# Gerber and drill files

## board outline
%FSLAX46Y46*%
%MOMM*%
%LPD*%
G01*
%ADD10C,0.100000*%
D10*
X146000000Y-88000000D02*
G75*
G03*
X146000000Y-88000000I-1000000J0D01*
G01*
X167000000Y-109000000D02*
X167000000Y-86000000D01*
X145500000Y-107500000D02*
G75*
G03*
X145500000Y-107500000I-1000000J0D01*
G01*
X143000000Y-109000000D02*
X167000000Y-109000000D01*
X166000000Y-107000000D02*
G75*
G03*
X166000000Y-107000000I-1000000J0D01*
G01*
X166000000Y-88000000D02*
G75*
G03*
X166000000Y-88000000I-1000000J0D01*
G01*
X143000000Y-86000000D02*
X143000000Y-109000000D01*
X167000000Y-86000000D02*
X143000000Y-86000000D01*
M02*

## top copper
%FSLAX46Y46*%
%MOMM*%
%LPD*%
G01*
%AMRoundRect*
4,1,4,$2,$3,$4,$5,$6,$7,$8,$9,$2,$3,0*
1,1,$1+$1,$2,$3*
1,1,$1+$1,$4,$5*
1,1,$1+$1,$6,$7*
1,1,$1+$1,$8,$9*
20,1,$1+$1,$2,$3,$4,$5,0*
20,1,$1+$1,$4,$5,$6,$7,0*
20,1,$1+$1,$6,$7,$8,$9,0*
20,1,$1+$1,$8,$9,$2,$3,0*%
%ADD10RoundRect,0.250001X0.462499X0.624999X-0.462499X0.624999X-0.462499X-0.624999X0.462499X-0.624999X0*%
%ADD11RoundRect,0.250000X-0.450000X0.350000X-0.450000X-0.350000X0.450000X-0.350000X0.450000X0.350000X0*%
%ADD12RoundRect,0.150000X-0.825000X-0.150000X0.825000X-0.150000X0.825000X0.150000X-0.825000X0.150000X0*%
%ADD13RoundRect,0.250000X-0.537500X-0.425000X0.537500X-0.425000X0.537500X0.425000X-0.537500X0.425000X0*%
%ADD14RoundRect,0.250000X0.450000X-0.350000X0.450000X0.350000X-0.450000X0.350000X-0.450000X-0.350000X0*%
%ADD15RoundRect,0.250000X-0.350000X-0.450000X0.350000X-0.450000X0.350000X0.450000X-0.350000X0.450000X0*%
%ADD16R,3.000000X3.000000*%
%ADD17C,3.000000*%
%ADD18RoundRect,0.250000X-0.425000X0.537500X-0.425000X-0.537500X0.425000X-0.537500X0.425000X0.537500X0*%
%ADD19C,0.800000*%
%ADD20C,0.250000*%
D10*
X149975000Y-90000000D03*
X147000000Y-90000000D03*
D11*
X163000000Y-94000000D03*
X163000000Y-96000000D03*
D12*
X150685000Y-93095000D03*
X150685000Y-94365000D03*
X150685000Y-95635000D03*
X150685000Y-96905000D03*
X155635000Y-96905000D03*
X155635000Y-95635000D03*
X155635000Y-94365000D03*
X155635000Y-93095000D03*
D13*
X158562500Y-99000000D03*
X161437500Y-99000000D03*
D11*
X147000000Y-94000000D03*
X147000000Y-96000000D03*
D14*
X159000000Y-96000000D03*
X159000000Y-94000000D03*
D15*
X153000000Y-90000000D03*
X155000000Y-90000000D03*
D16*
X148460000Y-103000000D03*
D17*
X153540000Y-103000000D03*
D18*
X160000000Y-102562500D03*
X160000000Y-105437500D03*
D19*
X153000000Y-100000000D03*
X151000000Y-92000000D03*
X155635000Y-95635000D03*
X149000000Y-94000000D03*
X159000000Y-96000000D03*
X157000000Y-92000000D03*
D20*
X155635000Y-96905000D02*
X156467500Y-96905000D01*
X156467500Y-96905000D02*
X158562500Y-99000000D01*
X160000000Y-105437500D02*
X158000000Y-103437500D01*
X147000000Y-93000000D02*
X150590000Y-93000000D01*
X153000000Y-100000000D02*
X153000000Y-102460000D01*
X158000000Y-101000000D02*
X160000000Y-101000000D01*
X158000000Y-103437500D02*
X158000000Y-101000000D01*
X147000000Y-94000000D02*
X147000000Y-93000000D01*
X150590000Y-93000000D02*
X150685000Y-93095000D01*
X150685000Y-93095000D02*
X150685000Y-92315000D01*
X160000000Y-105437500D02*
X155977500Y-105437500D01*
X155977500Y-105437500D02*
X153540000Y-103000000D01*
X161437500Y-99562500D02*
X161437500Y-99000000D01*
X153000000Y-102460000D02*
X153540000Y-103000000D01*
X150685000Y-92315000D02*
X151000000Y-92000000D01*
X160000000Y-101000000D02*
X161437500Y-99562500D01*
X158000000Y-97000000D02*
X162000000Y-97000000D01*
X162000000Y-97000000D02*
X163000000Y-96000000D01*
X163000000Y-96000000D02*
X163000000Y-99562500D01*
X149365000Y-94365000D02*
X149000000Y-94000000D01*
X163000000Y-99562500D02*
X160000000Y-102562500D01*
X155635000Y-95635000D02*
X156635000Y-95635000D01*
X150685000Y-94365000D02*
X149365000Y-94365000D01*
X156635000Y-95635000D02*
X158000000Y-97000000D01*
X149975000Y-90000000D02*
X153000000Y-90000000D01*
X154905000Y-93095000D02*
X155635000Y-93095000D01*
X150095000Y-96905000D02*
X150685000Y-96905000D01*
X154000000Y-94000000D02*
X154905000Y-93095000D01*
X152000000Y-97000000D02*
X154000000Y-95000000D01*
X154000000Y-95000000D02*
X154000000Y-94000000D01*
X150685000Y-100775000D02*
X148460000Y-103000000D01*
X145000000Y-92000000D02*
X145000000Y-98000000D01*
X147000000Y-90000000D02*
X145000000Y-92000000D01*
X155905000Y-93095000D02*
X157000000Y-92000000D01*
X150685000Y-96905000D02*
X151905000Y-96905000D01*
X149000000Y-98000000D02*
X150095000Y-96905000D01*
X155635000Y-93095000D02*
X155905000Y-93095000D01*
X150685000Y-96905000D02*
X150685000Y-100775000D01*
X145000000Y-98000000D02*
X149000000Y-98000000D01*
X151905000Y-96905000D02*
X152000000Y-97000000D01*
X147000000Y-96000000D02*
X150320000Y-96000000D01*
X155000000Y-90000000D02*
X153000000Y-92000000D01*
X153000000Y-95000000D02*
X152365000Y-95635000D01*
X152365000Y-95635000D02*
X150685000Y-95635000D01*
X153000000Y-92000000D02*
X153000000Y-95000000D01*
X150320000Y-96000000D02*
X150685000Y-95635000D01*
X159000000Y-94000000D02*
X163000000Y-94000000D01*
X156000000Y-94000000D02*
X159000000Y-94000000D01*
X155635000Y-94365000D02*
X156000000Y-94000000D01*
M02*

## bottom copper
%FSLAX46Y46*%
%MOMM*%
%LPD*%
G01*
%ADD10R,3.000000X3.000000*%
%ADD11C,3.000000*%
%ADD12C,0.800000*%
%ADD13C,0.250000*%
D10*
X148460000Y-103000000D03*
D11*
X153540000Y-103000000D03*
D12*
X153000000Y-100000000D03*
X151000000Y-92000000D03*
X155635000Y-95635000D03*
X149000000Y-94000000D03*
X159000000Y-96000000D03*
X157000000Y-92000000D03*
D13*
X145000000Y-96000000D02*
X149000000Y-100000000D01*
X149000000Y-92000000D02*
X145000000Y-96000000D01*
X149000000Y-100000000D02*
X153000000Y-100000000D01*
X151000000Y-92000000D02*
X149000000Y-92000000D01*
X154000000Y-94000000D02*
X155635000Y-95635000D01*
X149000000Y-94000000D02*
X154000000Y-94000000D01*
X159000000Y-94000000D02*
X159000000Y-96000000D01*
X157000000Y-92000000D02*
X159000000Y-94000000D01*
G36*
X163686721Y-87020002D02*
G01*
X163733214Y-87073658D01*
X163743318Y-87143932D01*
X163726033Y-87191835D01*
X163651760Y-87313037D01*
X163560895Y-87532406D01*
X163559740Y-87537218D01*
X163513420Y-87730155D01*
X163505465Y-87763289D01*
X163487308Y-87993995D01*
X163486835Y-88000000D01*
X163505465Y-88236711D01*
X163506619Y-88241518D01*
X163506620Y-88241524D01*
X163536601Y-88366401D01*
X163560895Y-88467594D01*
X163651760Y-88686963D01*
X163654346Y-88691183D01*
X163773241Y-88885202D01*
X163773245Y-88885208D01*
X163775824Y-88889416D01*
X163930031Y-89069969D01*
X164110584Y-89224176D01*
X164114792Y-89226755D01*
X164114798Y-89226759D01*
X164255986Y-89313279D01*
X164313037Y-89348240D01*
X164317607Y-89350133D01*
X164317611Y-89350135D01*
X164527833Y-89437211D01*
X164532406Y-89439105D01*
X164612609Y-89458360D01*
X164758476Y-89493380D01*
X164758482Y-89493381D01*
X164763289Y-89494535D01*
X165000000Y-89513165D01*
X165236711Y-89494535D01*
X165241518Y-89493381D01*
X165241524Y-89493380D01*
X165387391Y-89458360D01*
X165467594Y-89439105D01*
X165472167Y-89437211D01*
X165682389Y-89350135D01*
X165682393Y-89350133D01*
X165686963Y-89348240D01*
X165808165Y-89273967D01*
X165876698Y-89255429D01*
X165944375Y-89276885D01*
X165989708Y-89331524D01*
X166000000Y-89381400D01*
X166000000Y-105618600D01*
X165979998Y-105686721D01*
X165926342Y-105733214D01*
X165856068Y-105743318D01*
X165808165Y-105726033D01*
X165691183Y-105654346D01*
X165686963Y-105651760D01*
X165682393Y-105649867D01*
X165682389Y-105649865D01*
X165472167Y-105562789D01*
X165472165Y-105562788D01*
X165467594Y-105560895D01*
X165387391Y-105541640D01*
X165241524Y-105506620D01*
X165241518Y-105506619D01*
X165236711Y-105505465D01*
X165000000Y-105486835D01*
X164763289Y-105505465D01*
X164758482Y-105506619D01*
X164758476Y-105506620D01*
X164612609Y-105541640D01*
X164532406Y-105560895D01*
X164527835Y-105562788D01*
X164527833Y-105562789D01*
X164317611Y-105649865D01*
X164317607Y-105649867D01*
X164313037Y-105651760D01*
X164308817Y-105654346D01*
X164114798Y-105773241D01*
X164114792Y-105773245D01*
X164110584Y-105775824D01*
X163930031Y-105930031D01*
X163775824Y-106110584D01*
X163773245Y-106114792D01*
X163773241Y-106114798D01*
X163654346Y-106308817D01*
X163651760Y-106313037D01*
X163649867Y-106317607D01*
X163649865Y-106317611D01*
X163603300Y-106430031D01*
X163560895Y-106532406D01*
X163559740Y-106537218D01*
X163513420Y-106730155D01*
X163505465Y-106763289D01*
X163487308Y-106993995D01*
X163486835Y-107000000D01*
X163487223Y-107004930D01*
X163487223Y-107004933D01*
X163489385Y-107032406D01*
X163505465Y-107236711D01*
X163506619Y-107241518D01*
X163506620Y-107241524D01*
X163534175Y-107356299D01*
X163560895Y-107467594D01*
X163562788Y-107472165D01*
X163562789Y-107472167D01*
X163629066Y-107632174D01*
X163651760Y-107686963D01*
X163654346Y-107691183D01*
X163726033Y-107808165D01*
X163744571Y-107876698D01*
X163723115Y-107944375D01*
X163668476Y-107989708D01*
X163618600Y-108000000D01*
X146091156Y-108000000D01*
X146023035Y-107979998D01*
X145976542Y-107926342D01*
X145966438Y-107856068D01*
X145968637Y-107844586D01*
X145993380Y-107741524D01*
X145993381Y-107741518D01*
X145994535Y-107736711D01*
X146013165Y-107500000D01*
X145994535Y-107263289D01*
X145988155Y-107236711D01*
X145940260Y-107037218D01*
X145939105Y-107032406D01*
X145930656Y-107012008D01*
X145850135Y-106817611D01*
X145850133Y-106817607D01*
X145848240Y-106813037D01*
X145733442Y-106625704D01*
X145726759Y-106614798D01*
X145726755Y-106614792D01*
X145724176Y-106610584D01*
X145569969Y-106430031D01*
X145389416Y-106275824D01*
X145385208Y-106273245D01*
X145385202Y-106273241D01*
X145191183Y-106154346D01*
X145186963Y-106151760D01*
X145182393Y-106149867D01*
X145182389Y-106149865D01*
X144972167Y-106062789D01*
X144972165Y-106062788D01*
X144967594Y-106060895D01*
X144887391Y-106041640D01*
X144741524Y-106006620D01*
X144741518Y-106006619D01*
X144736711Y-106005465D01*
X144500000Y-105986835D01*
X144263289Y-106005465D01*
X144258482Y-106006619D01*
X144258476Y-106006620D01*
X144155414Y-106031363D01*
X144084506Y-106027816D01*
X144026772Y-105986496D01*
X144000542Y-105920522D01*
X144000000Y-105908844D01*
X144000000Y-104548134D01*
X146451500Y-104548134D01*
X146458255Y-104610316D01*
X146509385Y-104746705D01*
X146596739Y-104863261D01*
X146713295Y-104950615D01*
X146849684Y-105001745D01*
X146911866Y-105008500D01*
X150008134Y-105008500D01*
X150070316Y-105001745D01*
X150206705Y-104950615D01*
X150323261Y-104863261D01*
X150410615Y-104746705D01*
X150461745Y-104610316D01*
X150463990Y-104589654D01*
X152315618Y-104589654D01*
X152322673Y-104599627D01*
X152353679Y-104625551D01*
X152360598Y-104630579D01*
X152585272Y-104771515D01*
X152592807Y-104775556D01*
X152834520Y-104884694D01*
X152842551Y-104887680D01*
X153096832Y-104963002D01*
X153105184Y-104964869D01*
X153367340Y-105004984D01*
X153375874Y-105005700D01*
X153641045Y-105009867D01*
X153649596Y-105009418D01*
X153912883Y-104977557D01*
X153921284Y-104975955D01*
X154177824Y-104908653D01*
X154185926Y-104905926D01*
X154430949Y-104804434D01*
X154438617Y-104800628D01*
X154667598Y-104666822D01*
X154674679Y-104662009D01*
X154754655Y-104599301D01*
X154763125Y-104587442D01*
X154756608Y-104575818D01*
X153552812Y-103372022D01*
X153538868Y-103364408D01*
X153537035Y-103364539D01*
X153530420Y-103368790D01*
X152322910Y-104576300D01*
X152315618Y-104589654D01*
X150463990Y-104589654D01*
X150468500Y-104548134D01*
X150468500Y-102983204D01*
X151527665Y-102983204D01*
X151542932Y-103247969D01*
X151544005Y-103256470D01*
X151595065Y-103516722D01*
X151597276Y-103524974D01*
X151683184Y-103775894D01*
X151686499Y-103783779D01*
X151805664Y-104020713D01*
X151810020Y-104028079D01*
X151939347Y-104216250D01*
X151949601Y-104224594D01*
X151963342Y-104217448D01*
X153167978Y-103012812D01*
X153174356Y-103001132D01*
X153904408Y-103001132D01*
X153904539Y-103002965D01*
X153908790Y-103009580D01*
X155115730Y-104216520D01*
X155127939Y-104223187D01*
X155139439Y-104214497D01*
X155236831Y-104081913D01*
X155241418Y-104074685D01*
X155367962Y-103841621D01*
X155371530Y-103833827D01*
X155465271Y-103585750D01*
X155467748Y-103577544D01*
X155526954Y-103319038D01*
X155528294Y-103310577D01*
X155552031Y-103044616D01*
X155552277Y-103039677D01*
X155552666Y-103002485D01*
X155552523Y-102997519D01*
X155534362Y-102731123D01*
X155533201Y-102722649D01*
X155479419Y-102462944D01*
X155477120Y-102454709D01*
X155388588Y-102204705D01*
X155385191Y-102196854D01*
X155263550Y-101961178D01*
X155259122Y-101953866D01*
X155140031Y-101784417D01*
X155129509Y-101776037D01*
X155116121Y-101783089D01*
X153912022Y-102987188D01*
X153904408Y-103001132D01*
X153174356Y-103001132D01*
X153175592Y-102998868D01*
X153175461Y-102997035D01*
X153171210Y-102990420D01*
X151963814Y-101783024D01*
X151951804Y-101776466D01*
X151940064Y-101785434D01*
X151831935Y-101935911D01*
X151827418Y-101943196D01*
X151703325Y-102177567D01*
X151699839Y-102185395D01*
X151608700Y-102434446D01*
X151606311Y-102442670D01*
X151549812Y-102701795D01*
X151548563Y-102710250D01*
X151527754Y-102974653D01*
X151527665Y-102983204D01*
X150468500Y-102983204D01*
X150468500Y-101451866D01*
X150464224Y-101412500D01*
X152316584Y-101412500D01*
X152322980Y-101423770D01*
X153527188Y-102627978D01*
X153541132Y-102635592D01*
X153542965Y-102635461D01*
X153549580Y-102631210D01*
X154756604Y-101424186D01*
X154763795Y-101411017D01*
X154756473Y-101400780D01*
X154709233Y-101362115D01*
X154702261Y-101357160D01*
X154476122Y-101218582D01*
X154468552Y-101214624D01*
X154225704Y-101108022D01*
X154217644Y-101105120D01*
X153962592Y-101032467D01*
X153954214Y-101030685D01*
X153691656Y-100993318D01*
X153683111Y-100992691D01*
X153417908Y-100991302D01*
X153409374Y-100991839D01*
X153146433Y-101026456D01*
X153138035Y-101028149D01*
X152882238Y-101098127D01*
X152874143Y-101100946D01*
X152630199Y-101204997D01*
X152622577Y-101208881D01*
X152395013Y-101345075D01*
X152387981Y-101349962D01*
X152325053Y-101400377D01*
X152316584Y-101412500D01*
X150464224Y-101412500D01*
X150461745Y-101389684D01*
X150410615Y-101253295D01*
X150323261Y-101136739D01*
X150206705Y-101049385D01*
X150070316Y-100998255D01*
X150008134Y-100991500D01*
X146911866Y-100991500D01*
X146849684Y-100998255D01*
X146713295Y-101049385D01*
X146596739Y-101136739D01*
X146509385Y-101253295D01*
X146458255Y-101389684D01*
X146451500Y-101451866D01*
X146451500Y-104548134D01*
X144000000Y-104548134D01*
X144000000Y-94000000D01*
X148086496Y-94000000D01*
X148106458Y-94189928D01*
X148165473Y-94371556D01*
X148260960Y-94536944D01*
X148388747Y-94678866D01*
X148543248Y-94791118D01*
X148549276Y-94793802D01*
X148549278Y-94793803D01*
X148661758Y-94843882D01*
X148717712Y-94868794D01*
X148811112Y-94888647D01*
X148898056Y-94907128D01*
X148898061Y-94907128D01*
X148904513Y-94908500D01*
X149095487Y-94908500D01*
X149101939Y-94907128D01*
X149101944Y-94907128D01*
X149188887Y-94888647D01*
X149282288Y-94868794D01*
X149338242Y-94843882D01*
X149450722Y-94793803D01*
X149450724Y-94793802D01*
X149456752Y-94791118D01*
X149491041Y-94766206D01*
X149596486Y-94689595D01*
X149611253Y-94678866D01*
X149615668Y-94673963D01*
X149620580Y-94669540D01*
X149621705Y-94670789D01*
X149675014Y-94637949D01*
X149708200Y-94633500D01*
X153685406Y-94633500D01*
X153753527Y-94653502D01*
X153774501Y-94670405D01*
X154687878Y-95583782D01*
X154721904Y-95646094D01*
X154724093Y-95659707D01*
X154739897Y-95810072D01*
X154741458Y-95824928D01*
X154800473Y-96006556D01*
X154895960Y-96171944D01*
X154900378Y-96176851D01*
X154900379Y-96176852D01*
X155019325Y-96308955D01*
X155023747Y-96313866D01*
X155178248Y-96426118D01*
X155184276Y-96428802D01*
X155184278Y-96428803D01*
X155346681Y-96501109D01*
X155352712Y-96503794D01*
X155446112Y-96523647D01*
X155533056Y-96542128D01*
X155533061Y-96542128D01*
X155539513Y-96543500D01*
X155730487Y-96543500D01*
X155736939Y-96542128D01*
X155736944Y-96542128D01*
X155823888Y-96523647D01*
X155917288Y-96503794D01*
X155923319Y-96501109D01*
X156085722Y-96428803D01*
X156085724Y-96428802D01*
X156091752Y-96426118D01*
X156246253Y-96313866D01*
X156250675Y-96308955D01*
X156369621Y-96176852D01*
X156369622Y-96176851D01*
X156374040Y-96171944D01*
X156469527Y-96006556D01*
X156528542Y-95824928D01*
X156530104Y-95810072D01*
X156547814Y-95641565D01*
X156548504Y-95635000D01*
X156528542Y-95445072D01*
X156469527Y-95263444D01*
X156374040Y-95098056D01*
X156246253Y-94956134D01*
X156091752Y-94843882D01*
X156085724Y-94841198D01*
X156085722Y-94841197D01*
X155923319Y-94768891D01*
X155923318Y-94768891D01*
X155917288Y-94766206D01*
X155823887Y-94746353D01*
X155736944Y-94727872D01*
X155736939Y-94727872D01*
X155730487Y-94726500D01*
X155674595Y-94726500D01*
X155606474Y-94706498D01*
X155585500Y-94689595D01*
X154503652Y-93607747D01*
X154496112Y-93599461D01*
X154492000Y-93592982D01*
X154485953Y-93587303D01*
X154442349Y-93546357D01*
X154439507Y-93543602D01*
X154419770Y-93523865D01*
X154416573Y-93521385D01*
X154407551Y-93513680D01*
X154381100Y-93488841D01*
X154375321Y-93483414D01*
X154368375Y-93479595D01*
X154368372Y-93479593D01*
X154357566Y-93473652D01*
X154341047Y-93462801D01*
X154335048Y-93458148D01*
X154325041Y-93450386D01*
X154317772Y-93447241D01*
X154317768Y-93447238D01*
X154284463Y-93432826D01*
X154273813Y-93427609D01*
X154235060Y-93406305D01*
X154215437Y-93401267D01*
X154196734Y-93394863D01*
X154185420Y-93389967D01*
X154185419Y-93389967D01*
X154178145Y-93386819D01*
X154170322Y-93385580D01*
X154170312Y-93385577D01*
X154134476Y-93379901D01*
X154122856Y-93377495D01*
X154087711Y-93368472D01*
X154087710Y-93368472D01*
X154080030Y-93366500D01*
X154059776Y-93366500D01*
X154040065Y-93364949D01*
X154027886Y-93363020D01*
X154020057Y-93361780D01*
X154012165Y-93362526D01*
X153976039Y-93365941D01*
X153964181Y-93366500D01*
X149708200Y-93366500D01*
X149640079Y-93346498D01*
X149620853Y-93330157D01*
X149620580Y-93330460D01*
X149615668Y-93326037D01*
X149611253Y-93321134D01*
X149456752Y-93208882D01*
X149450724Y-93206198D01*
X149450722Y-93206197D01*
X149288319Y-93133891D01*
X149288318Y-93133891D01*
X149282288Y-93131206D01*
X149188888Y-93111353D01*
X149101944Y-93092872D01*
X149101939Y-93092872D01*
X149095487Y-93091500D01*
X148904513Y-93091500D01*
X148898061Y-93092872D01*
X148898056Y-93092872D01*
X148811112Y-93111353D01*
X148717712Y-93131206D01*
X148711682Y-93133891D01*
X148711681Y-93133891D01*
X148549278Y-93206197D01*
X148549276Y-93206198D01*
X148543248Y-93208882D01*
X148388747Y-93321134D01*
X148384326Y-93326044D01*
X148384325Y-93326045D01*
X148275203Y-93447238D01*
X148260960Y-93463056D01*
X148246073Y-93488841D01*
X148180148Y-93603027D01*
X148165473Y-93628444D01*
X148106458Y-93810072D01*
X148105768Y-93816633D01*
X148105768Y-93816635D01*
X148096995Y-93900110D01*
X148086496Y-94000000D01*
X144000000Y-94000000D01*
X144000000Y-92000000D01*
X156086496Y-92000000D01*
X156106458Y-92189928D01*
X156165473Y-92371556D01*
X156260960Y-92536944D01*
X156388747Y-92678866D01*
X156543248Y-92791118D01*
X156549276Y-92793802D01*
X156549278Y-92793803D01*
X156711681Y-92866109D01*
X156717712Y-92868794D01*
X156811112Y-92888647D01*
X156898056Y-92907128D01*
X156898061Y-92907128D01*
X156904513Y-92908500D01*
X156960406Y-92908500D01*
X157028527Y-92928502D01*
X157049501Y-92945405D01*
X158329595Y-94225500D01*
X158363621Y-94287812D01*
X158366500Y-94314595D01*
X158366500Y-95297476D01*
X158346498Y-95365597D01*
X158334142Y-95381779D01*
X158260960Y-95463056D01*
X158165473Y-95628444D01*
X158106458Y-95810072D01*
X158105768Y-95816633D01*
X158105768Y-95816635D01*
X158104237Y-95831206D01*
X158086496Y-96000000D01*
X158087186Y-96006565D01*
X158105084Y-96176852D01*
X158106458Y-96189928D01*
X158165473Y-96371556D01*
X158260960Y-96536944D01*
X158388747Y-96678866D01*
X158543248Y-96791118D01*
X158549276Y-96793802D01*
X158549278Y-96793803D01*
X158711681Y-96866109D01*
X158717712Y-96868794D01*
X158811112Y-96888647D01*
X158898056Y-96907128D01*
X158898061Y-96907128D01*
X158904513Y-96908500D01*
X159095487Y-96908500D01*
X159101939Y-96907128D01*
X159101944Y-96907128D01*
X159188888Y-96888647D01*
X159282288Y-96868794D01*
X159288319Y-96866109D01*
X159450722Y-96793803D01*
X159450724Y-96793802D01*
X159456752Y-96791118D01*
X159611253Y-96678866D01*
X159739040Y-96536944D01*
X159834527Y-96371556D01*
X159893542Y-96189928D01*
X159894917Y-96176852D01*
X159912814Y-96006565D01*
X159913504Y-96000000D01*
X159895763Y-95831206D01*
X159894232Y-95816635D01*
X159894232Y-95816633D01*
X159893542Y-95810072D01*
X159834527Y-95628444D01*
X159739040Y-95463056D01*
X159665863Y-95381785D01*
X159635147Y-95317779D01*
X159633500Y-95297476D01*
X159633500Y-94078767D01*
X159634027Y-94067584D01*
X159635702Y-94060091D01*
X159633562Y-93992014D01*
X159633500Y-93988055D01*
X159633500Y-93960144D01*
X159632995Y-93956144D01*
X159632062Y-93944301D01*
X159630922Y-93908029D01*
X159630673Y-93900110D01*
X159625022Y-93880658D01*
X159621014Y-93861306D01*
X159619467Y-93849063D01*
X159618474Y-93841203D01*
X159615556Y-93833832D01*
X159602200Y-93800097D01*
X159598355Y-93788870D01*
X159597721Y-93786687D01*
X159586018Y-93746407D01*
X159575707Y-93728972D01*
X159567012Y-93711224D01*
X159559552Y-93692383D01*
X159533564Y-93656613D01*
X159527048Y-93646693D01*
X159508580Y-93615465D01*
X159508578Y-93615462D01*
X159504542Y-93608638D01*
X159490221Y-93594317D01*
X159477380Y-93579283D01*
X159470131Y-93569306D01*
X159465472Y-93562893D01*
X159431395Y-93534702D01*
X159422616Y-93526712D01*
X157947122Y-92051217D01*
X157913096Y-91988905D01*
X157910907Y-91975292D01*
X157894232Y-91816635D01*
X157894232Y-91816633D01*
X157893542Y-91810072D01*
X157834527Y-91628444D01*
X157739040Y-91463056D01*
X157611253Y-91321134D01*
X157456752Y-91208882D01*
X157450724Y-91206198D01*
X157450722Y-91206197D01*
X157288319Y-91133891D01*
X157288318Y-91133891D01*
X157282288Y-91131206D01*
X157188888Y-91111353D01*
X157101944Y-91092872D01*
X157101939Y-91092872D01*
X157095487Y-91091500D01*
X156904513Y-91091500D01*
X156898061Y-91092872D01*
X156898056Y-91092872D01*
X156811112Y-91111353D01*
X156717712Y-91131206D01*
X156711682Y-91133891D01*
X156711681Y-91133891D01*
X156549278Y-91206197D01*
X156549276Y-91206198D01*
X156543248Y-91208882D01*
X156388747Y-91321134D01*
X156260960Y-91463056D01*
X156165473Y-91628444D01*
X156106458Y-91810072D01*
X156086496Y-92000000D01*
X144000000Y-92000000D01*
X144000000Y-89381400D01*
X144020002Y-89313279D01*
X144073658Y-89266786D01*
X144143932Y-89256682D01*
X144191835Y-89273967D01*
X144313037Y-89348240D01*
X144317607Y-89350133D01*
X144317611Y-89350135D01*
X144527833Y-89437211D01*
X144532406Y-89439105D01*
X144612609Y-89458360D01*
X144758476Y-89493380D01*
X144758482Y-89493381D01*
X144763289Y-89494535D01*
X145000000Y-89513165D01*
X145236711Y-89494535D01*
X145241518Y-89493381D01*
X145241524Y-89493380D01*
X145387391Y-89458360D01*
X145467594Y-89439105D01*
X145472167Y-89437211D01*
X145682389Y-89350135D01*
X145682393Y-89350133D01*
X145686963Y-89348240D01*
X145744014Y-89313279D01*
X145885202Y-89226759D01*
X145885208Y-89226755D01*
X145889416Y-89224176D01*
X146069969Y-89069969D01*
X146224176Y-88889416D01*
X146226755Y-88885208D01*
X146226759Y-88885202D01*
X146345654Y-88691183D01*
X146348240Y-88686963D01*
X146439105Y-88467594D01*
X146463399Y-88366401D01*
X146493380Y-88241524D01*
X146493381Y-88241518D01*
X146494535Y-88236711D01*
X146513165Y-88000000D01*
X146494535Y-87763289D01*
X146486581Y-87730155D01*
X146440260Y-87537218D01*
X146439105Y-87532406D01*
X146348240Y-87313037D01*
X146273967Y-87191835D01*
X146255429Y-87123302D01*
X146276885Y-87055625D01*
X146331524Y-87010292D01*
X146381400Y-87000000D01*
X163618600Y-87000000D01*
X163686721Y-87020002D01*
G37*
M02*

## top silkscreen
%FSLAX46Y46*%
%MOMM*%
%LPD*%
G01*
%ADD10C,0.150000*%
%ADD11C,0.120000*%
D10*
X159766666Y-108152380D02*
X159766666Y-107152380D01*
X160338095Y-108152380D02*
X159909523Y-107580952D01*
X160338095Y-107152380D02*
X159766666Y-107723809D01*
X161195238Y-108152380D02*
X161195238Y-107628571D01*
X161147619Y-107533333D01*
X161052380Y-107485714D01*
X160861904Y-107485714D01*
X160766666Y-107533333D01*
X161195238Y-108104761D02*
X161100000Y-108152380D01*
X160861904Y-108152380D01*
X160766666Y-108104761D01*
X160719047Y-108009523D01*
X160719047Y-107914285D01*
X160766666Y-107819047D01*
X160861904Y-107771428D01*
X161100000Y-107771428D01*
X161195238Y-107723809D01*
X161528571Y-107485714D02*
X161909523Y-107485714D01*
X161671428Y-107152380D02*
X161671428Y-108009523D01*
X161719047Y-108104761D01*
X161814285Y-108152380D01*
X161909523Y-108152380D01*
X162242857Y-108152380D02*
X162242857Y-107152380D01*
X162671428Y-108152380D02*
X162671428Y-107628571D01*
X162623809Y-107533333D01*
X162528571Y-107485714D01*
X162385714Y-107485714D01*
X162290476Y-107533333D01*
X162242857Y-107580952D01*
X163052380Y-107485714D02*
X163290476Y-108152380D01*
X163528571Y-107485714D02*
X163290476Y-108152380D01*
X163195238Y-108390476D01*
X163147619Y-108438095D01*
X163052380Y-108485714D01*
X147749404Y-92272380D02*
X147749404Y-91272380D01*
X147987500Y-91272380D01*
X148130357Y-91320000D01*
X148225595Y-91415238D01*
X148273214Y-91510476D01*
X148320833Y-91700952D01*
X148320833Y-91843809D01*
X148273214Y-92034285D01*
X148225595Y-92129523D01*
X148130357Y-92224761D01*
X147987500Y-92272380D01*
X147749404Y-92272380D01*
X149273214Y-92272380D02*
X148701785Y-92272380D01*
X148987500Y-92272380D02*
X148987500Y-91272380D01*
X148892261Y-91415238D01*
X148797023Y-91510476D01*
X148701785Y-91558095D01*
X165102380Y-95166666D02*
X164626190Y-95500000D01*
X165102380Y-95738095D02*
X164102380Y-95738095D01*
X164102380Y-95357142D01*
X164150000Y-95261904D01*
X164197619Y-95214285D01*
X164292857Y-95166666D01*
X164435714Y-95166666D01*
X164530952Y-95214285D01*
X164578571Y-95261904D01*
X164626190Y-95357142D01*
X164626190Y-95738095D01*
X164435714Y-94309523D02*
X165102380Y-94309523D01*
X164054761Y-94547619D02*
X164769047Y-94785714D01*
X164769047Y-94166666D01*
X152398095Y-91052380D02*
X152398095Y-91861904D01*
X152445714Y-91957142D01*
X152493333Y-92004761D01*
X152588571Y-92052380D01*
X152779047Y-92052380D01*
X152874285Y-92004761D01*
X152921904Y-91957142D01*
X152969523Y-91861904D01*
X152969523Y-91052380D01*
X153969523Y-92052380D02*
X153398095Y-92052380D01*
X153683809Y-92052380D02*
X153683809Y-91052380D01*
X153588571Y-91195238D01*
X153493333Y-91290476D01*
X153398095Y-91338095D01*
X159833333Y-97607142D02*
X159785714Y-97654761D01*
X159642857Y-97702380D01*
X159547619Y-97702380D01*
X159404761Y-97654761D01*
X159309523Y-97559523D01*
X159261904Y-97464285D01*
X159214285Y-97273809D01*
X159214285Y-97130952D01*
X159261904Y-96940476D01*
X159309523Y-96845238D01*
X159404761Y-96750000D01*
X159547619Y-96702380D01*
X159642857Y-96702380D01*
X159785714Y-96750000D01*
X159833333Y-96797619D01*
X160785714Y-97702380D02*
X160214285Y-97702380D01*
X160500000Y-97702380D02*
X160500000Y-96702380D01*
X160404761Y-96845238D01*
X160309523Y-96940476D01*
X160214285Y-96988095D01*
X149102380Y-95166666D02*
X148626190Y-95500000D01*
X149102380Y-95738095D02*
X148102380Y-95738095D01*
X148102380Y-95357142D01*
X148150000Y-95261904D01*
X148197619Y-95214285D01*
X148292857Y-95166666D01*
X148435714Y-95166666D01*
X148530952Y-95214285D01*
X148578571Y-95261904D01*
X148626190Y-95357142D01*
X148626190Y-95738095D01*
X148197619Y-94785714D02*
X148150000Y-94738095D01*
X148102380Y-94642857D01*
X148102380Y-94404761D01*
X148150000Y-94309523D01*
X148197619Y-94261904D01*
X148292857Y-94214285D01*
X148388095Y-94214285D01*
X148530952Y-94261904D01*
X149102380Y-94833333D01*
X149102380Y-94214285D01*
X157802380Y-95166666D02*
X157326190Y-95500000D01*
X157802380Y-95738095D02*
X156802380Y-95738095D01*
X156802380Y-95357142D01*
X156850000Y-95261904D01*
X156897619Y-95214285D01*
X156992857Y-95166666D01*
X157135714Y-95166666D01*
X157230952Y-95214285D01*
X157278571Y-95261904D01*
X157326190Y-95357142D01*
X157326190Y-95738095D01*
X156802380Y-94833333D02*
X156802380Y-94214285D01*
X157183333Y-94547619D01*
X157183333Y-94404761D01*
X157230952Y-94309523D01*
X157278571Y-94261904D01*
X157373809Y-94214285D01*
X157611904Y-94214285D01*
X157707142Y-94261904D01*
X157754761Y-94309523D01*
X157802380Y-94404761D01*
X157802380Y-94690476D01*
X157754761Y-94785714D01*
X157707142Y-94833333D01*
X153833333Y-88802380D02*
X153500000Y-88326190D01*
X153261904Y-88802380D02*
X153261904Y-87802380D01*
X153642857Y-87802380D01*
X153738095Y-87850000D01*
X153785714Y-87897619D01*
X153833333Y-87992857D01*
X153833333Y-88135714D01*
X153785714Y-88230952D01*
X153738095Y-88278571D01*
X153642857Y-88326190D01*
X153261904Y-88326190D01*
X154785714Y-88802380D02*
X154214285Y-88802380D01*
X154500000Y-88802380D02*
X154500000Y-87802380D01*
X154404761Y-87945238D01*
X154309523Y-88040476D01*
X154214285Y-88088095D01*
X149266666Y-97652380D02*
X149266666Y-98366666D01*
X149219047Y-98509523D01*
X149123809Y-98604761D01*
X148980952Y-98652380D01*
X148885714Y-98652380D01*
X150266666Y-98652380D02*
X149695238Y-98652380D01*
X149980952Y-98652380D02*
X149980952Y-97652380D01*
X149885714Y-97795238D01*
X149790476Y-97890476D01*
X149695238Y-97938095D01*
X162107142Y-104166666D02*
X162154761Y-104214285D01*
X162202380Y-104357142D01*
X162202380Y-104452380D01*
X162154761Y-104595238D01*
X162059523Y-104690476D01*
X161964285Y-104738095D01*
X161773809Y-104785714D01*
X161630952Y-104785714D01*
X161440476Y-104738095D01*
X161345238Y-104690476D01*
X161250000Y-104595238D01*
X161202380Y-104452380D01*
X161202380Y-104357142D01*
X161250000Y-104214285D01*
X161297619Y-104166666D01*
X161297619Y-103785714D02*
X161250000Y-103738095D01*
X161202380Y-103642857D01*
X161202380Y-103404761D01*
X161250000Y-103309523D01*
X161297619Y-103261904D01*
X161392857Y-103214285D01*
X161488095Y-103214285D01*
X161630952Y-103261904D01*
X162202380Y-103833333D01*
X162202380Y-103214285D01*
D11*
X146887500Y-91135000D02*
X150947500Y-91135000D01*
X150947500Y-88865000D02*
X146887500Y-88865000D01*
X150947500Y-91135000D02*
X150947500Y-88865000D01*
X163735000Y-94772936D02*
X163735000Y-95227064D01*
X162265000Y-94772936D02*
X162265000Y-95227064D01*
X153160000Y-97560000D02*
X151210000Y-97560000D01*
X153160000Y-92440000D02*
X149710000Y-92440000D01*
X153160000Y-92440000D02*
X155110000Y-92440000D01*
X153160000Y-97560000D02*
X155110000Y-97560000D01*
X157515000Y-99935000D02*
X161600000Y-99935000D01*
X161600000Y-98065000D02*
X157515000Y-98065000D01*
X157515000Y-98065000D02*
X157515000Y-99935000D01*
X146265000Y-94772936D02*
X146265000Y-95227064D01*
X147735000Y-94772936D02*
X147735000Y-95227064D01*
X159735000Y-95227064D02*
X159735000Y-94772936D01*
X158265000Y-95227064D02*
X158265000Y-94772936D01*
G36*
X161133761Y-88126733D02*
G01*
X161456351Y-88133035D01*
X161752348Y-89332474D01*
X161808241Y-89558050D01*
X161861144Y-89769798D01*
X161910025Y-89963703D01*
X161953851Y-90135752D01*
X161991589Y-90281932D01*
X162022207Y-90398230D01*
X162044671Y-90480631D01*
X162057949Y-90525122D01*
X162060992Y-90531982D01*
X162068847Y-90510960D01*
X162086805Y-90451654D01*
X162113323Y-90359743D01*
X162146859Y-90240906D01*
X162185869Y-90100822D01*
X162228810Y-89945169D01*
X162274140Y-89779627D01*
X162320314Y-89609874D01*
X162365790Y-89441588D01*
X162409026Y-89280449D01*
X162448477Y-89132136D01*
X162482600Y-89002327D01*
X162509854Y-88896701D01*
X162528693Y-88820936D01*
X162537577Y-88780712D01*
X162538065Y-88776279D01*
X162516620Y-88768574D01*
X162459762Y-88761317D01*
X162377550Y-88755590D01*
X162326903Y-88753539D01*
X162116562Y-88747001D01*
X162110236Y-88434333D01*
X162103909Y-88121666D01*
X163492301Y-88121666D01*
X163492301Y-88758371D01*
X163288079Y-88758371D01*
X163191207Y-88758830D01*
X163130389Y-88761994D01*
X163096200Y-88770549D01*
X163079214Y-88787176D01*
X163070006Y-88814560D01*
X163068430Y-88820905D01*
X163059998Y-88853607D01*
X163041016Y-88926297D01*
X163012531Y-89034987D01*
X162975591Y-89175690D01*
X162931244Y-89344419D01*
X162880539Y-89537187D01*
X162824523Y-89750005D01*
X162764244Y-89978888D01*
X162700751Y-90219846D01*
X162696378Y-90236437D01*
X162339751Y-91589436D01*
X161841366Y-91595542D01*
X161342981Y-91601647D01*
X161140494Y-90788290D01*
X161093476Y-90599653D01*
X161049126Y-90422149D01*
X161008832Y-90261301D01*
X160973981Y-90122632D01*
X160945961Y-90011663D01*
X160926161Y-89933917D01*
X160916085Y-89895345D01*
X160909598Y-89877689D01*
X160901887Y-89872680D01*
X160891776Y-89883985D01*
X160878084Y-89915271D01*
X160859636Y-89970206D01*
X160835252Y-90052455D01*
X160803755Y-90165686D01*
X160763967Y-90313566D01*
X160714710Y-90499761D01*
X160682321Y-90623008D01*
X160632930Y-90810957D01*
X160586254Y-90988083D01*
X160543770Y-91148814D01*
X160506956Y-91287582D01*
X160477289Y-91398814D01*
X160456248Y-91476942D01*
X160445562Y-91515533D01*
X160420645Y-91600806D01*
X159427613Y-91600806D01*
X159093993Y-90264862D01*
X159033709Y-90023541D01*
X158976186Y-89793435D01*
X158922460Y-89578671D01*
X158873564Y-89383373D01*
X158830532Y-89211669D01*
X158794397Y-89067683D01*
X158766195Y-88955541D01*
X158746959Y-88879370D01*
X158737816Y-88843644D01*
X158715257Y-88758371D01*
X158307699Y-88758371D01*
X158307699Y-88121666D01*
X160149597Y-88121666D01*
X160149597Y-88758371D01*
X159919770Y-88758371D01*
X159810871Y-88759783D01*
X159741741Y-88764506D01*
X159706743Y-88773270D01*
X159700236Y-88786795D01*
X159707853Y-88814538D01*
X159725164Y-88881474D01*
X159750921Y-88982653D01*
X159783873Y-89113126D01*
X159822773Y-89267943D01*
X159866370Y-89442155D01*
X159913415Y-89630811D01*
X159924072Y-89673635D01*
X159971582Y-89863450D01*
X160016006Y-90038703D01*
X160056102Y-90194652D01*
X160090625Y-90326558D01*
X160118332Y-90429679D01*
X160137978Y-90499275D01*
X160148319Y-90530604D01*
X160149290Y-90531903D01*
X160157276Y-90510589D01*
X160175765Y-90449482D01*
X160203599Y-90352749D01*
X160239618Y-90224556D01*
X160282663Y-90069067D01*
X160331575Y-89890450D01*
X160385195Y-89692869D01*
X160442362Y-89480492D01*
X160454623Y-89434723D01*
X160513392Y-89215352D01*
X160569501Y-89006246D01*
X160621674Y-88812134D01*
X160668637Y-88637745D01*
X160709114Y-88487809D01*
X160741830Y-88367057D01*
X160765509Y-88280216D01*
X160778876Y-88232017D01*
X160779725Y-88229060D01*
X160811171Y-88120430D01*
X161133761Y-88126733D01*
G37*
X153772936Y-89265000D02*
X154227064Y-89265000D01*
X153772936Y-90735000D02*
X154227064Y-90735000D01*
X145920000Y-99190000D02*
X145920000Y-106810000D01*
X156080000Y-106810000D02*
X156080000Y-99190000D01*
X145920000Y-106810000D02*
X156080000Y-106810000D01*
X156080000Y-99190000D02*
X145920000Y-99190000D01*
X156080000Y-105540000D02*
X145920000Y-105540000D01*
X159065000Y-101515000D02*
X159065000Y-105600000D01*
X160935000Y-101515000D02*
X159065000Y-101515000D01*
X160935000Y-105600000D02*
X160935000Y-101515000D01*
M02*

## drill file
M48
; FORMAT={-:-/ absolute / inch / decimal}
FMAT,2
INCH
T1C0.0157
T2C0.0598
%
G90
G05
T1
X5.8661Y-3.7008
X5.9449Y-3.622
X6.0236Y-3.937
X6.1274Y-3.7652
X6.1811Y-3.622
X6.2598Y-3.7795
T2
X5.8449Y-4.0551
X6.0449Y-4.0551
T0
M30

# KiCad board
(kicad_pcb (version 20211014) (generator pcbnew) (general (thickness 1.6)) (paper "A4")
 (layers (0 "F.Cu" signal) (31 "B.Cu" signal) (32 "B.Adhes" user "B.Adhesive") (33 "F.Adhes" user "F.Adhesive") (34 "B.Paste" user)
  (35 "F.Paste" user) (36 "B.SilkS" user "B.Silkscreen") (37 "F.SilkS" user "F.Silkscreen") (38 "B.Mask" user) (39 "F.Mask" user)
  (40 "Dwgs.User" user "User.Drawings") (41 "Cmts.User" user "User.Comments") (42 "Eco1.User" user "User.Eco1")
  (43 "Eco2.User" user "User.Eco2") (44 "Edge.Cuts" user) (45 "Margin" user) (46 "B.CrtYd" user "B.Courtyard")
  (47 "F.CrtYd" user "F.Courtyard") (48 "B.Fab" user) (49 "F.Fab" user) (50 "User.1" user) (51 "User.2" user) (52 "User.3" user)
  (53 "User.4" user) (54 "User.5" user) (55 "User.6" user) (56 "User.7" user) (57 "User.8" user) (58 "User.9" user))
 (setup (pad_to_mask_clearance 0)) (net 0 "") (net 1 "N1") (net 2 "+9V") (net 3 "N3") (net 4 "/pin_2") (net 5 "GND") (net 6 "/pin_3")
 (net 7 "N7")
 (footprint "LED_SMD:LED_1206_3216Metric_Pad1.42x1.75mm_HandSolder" (layer "F.Cu") (at 148.4875 90 180)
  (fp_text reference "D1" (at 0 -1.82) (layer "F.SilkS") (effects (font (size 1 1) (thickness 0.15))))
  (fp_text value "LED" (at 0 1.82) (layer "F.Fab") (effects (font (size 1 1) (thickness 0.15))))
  (fp_line (start 1.6 -1.135) (end -2.46 -1.135) (layer "F.SilkS") (width 0.12))
  (fp_line (start -2.46 1.135) (end 1.6 1.135) (layer "F.SilkS") (width 0.12))
  (fp_line (start -2.46 -1.135) (end -2.46 1.135) (layer "F.SilkS") (width 0.12))
  (pad "1" smd roundrect (at -1.4875 0 180) (size 1.425 1.75) (layers "F.Cu" "F.Paste" "F.Mask") (roundrect_rratio 0.1754392982)
   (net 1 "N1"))
  (pad "2" smd roundrect (at 1.4875 0 180) (size 1.425 1.75) (layers "F.Cu" "F.Paste" "F.Mask") (roundrect_rratio 0.1754392982)
   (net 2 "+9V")))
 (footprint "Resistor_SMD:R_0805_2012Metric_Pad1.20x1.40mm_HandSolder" (layer "F.Cu") (at 163 95 -90)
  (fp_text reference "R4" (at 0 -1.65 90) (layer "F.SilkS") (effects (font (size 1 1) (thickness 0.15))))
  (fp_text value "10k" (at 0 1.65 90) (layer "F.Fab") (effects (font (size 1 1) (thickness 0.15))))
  (fp_line (start -0.227064 -0.735) (end 0.227064 -0.735) (layer "F.SilkS") (width 0.12))
  (fp_line (start -0.227064 0.735) (end 0.227064 0.735) (layer "F.SilkS") (width 0.12))
  (pad "1" smd roundrect (at -1 0 270) (size 1.2 1.4) (layers "F.Cu" "F.Paste" "F.Mask") (roundrect_rratio 0.2083333333) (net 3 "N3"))
  (pad "2" smd roundrect (at 1 0 270) (size 1.2 1.4) (layers "F.Cu" "F.Paste" "F.Mask") (roundrect_rratio 0.2083333333) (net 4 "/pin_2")))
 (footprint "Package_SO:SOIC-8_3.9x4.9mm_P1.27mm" (layer "F.Cu") (at 153.16 95)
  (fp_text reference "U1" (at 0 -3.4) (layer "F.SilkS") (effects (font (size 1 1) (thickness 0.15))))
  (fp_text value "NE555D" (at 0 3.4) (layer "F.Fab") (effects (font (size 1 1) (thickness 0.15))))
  (fp_line (start 0 2.56) (end -1.95 2.56) (layer "F.SilkS") (width 0.12))
  (fp_line (start 0 -2.56) (end -3.45 -2.56) (layer "F.SilkS") (width 0.12))
  (fp_line (start 0 -2.56) (end 1.95 -2.56) (layer "F.SilkS") (width 0.12))
  (fp_line (start 0 2.56) (end 1.95 2.56) (layer "F.SilkS") (width 0.12))
  (pad "1" smd roundrect (at -2.475 -1.905) (size 1.95 0.6) (layers "F.Cu" "F.Paste" "F.Mask") (roundrect_rratio 0.25) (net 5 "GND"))
  (pad "2" smd roundrect (at -2.475 -0.635) (size 1.95 0.6) (layers "F.Cu" "F.Paste" "F.Mask") (roundrect_rratio 0.25) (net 4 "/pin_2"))
  (pad "3" smd roundrect (at -2.475 0.635) (size 1.95 0.6) (layers "F.Cu" "F.Paste" "F.Mask") (roundrect_rratio 0.25) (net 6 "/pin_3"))
  (pad "4" smd roundrect (at -2.475 1.905) (size 1.95 0.6) (layers "F.Cu" "F.Paste" "F.Mask") (roundrect_rratio 0.25) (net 2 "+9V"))
  (pad "5" smd roundrect (at 2.475 1.905) (size 1.95 0.6) (layers "F.Cu" "F.Paste" "F.Mask") (roundrect_rratio 0.25) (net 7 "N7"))
  (pad "6" smd roundrect (at 2.475 0.635) (size 1.95 0.6) (layers "F.Cu" "F.Paste" "F.Mask") (roundrect_rratio 0.25) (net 4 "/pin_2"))
  (pad "7" smd roundrect (at 2.475 -0.635) (size 1.95 0.6) (layers "F.Cu" "F.Paste" "F.Mask") (roundrect_rratio 0.25) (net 3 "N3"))
  (pad "8" smd roundrect (at 2.475 -1.905) (size 1.95 0.6) (layers "F.Cu" "F.Paste" "F.Mask") (roundrect_rratio 0.25) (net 2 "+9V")))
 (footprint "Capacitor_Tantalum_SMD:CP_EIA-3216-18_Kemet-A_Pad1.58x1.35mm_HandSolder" (layer "F.Cu") (at 160 99)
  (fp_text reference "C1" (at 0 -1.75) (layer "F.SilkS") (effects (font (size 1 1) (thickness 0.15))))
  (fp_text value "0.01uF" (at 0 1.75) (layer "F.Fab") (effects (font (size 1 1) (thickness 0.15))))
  (fp_line (start -2.485 0.935) (end 1.6 0.935) (layer "F.SilkS") (width 0.12))
  (fp_line (start 1.6 -0.935) (end -2.485 -0.935) (layer "F.SilkS") (width 0.12))
  (fp_line (start -2.485 -0.935) (end -2.485 0.935) (layer "F.SilkS") (width 0.12))
  (pad "1" smd roundrect (at -1.4375 0) (size 1.575 1.35) (layers "F.Cu" "F.Paste" "F.Mask") (roundrect_rratio 0.1851851852) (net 7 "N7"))
  (pad "2" smd roundrect (at 1.4375 0) (size 1.575 1.35) (layers "F.Cu" "F.Paste" "F.Mask") (roundrect_rratio 0.1851851852) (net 5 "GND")))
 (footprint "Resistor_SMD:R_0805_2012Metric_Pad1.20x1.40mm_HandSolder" (layer "F.Cu") (at 147 95 -90)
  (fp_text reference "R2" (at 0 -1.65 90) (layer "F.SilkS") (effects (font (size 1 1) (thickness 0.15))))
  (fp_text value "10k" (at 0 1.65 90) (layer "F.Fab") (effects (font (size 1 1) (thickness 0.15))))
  (fp_line (start -0.227064 0.735) (end 0.227064 0.735) (layer "F.SilkS") (width 0.12))
  (fp_line (start -0.227064 -0.735) (end 0.227064 -0.735) (layer "F.SilkS") (width 0.12))
  (pad "1" smd roundrect (at -1 0 270) (size 1.2 1.4) (layers "F.Cu" "F.Paste" "F.Mask") (roundrect_rratio 0.2083333333) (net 5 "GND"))
  (pad "2" smd roundrect (at 1 0 270) (size 1.2 1.4) (layers "F.Cu" "F.Paste" "F.Mask") (roundrect_rratio 0.2083333333) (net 6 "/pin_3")))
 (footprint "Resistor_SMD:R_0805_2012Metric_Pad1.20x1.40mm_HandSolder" (layer "F.Cu") (at 159 95 90)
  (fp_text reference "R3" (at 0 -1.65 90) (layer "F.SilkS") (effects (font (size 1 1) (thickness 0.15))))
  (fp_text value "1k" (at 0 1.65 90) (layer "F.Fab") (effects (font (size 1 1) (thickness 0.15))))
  (fp_line (start -0.227064 0.735) (end 0.227064 0.735) (layer "F.SilkS") (width 0.12))
  (fp_line (start -0.227064 -0.735) (end 0.227064 -0.735) (layer "F.SilkS") (width 0.12))
  (pad "1" smd roundrect (at -1 0 90) (size 1.2 1.4) (layers "F.Cu" "F.Paste" "F.Mask") (roundrect_rratio 0.2083333333) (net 2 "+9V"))
  (pad "2" smd roundrect (at 1 0 90) (size 1.2 1.4) (layers "F.Cu" "F.Paste" "F.Mask") (roundrect_rratio 0.2083333333) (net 3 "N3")))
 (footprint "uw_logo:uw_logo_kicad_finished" (layer "F.Cu") (at 160.9 90.1)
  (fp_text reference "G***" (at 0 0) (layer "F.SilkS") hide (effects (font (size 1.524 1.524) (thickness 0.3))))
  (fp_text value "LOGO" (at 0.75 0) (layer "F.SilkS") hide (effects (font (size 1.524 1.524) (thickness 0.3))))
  (fp_poly
   (pts (xy 0.233761 -1.973267) (xy 0.556351 -1.966965) (xy 0.852348 -0.767526) (xy 0.908241 -0.54195) (xy 0.961144 -0.330202)
    (xy 1.010025 -0.136297) (xy 1.053851 0.035752) (xy 1.091589 0.181932) (xy 1.122207 0.29823) (xy 1.144671 0.380631)
    (xy 1.157949 0.425122) (xy 1.160992 0.431982) (xy 1.168847 0.41096) (xy 1.186805 0.351654) (xy 1.213323 0.259743) (xy 1.246859 0.140906)
    (xy 1.285869 0.000822) (xy 1.32881 -0.154831) (xy 1.37414 -0.320373) (xy 1.420314 -0.490126) (xy 1.46579 -0.658412)
    (xy 1.509026 -0.819551) (xy 1.548477 -0.967864) (xy 1.5826 -1.097673) (xy 1.609854 -1.203299) (xy 1.628693 -1.279064)
    (xy 1.637577 -1.319288) (xy 1.638065 -1.323721) (xy 1.61662 -1.331426) (xy 1.559762 -1.338683) (xy 1.47755 -1.34441)
    (xy 1.426903 -1.346461) (xy 1.216562 -1.352999) (xy 1.210236 -1.665667) (xy 1.203909 -1.978334) (xy 2.592301 -1.978334)
    (xy 2.592301 -1.341629) (xy 2.388079 -1.341629) (xy 2.291207 -1.34117) (xy 2.230389 -1.338006) (xy 2.1962 -1.329451)
    (xy 2.179214 -1.312824) (xy 2.170006 -1.28544) (xy 2.16843 -1.279095) (xy 2.159998 -1.246393) (xy 2.141016 -1.173703)
    (xy 2.112531 -1.065013) (xy 2.075591 -0.92431) (xy 2.031244 -0.755581) (xy 1.980539 -0.562813) (xy 1.924523 -0.349995)
    (xy 1.864244 -0.121112) (xy 1.800751 0.119846) (xy 1.796378 0.136437) (xy 1.439751 1.489436) (xy 0.941366 1.495542)
    (xy 0.442981 1.501647) (xy 0.240494 0.68829) (xy 0.193476 0.499653) (xy 0.149126 0.322149) (xy 0.108832 0.161301) (xy 0.073981 0.022632)
    (xy 0.045961 -0.088337) (xy 0.026161 -0.166083) (xy 0.016085 -0.204655) (xy 0.009598 -0.222311) (xy 0.001887 -0.22732)
    (xy -0.008224 -0.216015) (xy -0.021916 -0.184729) (xy -0.040364 -0.129794) (xy -0.064748 -0.047545) (xy -0.096245 0.065686)
    (xy -0.136033 0.213566) (xy -0.18529 0.399761) (xy -0.217679 0.523008) (xy -0.26707 0.710957) (xy -0.313746 0.888083)
    (xy -0.35623 1.048814) (xy -0.393044 1.187582) (xy -0.422711 1.298814) (xy -0.443752 1.376942) (xy -0.454438 1.415533)
    (xy -0.479355 1.500806) (xy -1.472387 1.500806) (xy -1.806007 0.164862) (xy -1.866291 -0.076459) (xy -1.923814 -0.306565)
    (xy -1.97754 -0.521329) (xy -2.026436 -0.716627) (xy -2.069468 -0.888331) (xy -2.105603 -1.032317) (xy -2.133805 -1.144459)
    (xy -2.153041 -1.22063) (xy -2.162184 -1.256356) (xy -2.184743 -1.341629) (xy -2.592301 -1.341629) (xy -2.592301 -1.978334)
    (xy -0.750403 -1.978334) (xy -0.750403 -1.341629) (xy -0.98023 -1.341629) (xy -1.089129 -1.340217) (xy -1.158259 -1.335494)
    (xy -1.193257 -1.32673) (xy -1.199764 -1.313205) (xy -1.192147 -1.285462) (xy -1.174836 -1.218526) (xy -1.149079 -1.117347)
    (xy -1.116127 -0.986874) (xy -1.077227 -0.832057) (xy -1.03363 -0.657845) (xy -0.986585 -0.469189) (xy -0.975928 -0.426365)
    (xy -0.928418 -0.23655) (xy -0.883994 -0.061297) (xy -0.843898 0.094652) (xy -0.809375 0.226558) (xy -0.781668 0.329679)
    (xy -0.762022 0.399275) (xy -0.751681 0.430604) (xy -0.75071 0.431903) (xy -0.742724 0.410589) (xy -0.724235 0.349482)
    (xy -0.696401 0.252749) (xy -0.660382 0.124556) (xy -0.617337 -0.030933) (xy -0.568425 -0.20955) (xy -0.514805 -0.407131)
    (xy -0.457638 -0.619508) (xy -0.445377 -0.665277) (xy -0.386608 -0.884648) (xy -0.330499 -1.093754) (xy -0.278326 -1.287866)
    (xy -0.231363 -1.462255) (xy -0.190886 -1.612191) (xy -0.15817 -1.732943) (xy -0.134491 -1.819784) (xy -0.121124 -1.867983)
    (xy -0.120275 -1.87094) (xy -0.088829 -1.97957))
   (layer "F.SilkS") (width 0) (fill solid)))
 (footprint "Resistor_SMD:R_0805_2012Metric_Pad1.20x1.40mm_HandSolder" (layer "F.Cu") (at 154 90)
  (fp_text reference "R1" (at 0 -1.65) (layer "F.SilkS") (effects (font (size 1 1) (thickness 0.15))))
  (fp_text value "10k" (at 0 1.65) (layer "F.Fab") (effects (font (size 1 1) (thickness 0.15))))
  (fp_line (start -0.227064 -0.735) (end 0.227064 -0.735) (layer "F.SilkS") (width 0.12))
  (fp_line (start -0.227064 0.735) (end 0.227064 0.735) (layer "F.SilkS") (width 0.12))
  (pad "1" smd roundrect (at -1 0) (size 1.2 1.4) (layers "F.Cu" "F.Paste" "F.Mask") (roundrect_rratio 0.2083333333) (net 1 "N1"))
  (pad "2" smd roundrect (at 1 0) (size 1.2 1.4) (layers "F.Cu" "F.Paste" "F.Mask") (roundrect_rratio 0.2083333333) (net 6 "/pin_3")))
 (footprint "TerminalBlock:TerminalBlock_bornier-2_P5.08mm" (layer "F.Cu") (at 148.46 103)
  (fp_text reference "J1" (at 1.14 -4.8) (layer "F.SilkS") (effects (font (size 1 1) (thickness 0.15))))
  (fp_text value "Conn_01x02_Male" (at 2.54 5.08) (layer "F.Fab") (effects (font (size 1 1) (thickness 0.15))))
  (fp_line (start -2.54 -3.81) (end -2.54 3.81) (layer "F.SilkS") (width 0.12))
  (fp_line (start 7.62 3.81) (end 7.62 -3.81) (layer "F.SilkS") (width 0.12))
  (fp_line (start -2.54 3.81) (end 7.62 3.81) (layer "F.SilkS") (width 0.12))
  (fp_line (start 7.62 -3.81) (end -2.54 -3.81) (layer "F.SilkS") (width 0.12))
  (fp_line (start 7.62 2.54) (end -2.54 2.54) (layer "F.SilkS") (width 0.12))
  (pad "1" thru_hole rect (at 0 0) (size 3 3) (drill 1.52) (layers *.Cu *.Mask) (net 2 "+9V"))
  (pad "2" thru_hole circle (at 5.08 0) (size 3 3) (drill 1.52) (layers *.Cu *.Mask) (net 5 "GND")))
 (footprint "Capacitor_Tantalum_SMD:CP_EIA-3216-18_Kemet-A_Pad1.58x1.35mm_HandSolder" (layer "F.Cu") (at 160 104 -90)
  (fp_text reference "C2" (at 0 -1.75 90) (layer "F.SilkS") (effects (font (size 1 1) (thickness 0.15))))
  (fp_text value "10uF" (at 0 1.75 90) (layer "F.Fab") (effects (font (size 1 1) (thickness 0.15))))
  (fp_line (start -2.485 0.935) (end 1.6 0.935) (layer "F.SilkS") (width 0.12))
  (fp_line (start -2.485 -0.935) (end -2.485 0.935) (layer "F.SilkS") (width 0.12))
  (fp_line (start 1.6 -0.935) (end -2.485 -0.935) (layer "F.SilkS") (width 0.12))
  (pad "1" smd roundrect (at -1.4375 0 270) (size 1.575 1.35) (layers "F.Cu" "F.Paste" "F.Mask") (roundrect_rratio 0.1851851852)
   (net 4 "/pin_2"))
  (pad "2" smd roundrect (at 1.4375 0 270) (size 1.575 1.35) (layers "F.Cu" "F.Paste" "F.Mask") (roundrect_rratio 0.1851851852)
   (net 5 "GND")))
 (gr_circle (center 145 88) (end 144 88) (layer "Edge.Cuts") (width 0.1) (fill none))
 (gr_line (start 167 109) (end 167 86) (layer "Edge.Cuts") (width 0.1))
 (gr_circle (center 144.5 107.5) (end 145.5 107.5) (layer "Edge.Cuts") (width 0.1) (fill none))
 (gr_line (start 143 109) (end 167 109) (layer "Edge.Cuts") (width 0.1))
 (gr_circle (center 165 107) (end 166 107) (layer "Edge.Cuts") (width 0.1) (fill none))
 (gr_circle (center 165 88) (end 165 89) (layer "Edge.Cuts") (width 0.1) (fill none))
 (gr_line (start 143 86) (end 143 109) (layer "Edge.Cuts") (width 0.1))
 (gr_line (start 167 86) (end 143 86) (layer "Edge.Cuts") (width 0.1))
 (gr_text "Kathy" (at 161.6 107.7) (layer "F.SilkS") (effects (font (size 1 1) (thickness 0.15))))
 (segment (start 155.635 96.905) (end 156.4675 96.905) (width 0.25) (layer "F.Cu") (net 7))
 (segment (start 156.4675 96.905) (end 158.5625 99) (width 0.25) (layer "F.Cu") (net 7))
 (segment (start 160 105.4375) (end 158 103.4375) (width 0.25) (layer "F.Cu") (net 5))
 (segment (start 147 93) (end 150.59 93) (width 0.25) (layer "F.Cu") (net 5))
 (segment (start 153 100) (end 153 102.46) (width 0.25) (layer "F.Cu") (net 5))
 (segment (start 158 101) (end 160 101) (width 0.25) (layer "F.Cu") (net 5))
 (segment (start 158 103.4375) (end 158 101) (width 0.25) (layer "F.Cu") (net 5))
 (segment (start 147 94) (end 147 93) (width 0.25) (layer "F.Cu") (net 5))
 (segment (start 150.59 93) (end 150.685 93.095) (width 0.25) (layer "F.Cu") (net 5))
 (segment (start 150.685 93.095) (end 150.685 92.315) (width 0.25) (layer "F.Cu") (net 5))
 (segment (start 160 105.4375) (end 155.9775 105.4375) (width 0.25) (layer "F.Cu") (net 5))
 (segment (start 155.9775 105.4375) (end 153.54 103) (width 0.25) (layer "F.Cu") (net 5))
 (segment (start 161.4375 99.5625) (end 161.4375 99) (width 0.25) (layer "F.Cu") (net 5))
 (segment (start 153 102.46) (end 153.54 103) (width 0.25) (layer "F.Cu") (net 5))
 (segment (start 150.685 92.315) (end 151 92) (width 0.25) (layer "F.Cu") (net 5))
 (segment (start 160 101) (end 161.4375 99.5625) (width 0.25) (layer "F.Cu") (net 5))
 (via (at 153 100) (size 0.8) (drill 0.4) (layers "F.Cu" "B.Cu") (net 5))
 (via (at 151 92) (size 0.8) (drill 0.4) (layers "F.Cu" "B.Cu") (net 5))
 (segment (start 145 96) (end 149 100) (width 0.25) (layer "B.Cu") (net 5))
 (segment (start 149 92) (end 145 96) (width 0.25) (layer "B.Cu") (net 5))
 (segment (start 149 100) (end 153 100) (width 0.25) (layer "B.Cu") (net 5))
 (segment (start 151 92) (end 149 92) (width 0.25) (layer "B.Cu") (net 5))
 (segment (start 158 97) (end 162 97) (width 0.25) (layer "F.Cu") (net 4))
 (segment (start 162 97) (end 163 96) (width 0.25) (layer "F.Cu") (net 4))
 (segment (start 163 96) (end 163 99.5625) (width 0.25) (layer "F.Cu") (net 4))
 (segment (start 149.365 94.365) (end 149 94) (width 0.25) (layer "F.Cu") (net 4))
 (segment (start 163 99.5625) (end 160 102.5625) (width 0.25) (layer "F.Cu") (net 4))
 (segment (start 155.635 95.635) (end 156.635 95.635) (width 0.25) (layer "F.Cu") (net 4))
 (segment (start 150.685 94.365) (end 149.365 94.365) (width 0.25) (layer "F.Cu") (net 4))
 (segment (start 156.635 95.635) (end 158 97) (width 0.25) (layer "F.Cu") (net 4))
 (via (at 155.635 95.635) (size 0.8) (drill 0.4) (layers "F.Cu" "B.Cu") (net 4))
 (via (at 149 94) (size 0.8) (drill 0.4) (layers "F.Cu" "B.Cu") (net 4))
 (segment (start 154 94) (end 155.635 95.635) (width 0.25) (layer "B.Cu") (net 4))
 (segment (start 149 94) (end 154 94) (width 0.25) (layer "B.Cu") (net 4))
 (segment (start 149.975 90) (end 153 90) (width 0.25) (layer "F.Cu") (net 1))
 (segment (start 154.905 93.095) (end 155.635 93.095) (width 0.25) (layer "F.Cu") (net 2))
 (segment (start 150.095 96.905) (end 150.685 96.905) (width 0.25) (layer "F.Cu") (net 2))
 (segment (start 154 94) (end 154.905 93.095) (width 0.25) (layer "F.Cu") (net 2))
 (segment (start 152 97) (end 154 95) (width 0.25) (layer "F.Cu") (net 2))
 (segment (start 154 95) (end 154 94) (width 0.25) (layer "F.Cu") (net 2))
 (segment (start 150.685 100.775) (end 148.46 103) (width 0.25) (layer "F.Cu") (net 2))
 (segment (start 145 92) (end 145 98) (width 0.25) (layer "F.Cu") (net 2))
 (segment (start 147 90) (end 145 92) (width 0.25) (layer "F.Cu") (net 2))
 (segment (start 155.905 93.095) (end 157 92) (width 0.25) (layer "F.Cu") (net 2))
 (segment (start 150.685 96.905) (end 151.905 96.905) (width 0.25) (layer "F.Cu") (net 2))
 (segment (start 149 98) (end 150.095 96.905) (width 0.25) (layer "F.Cu") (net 2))
 (segment (start 155.635 93.095) (end 155.905 93.095) (width 0.25) (layer "F.Cu") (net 2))
 (segment (start 150.685 96.905) (end 150.685 100.775) (width 0.25) (layer "F.Cu") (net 2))
 (segment (start 145 98) (end 149 98) (width 0.25) (layer "F.Cu") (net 2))
 (segment (start 151.905 96.905) (end 152 97) (width 0.25) (layer "F.Cu") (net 2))
 (via (at 159 96) (size 0.8) (drill 0.4) (layers "F.Cu" "B.Cu") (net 2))
 (via (at 157 92) (size 0.8) (drill 0.4) (layers "F.Cu" "B.Cu") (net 2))
 (segment (start 159 94) (end 159 96) (width 0.25) (layer "B.Cu") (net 2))
 (segment (start 157 92) (end 159 94) (width 0.25) (layer "B.Cu") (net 2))
 (segment (start 147 96) (end 150.32 96) (width 0.25) (layer "F.Cu") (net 6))
 (segment (start 155 90) (end 153 92) (width 0.25) (layer "F.Cu") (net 6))
 (segment (start 153 95) (end 152.365 95.635) (width 0.25) (layer "F.Cu") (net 6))
 (segment (start 152.365 95.635) (end 150.685 95.635) (width 0.25) (layer "F.Cu") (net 6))
 (segment (start 153 92) (end 153 95) (width 0.25) (layer "F.Cu") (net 6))
 (segment (start 150.32 96) (end 150.685 95.635) (width 0.25) (layer "F.Cu") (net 6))
 (segment (start 159 94) (end 163 94) (width 0.25) (layer "F.Cu") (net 3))
 (segment (start 156 94) (end 159 94) (width 0.25) (layer "F.Cu") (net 3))
 (segment (start 155.635 94.365) (end 156 94) (width 0.25) (layer "F.Cu") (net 3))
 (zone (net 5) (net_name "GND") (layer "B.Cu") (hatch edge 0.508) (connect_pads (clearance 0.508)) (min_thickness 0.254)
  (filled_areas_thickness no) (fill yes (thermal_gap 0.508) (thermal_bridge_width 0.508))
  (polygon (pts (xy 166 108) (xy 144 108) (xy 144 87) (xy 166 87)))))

